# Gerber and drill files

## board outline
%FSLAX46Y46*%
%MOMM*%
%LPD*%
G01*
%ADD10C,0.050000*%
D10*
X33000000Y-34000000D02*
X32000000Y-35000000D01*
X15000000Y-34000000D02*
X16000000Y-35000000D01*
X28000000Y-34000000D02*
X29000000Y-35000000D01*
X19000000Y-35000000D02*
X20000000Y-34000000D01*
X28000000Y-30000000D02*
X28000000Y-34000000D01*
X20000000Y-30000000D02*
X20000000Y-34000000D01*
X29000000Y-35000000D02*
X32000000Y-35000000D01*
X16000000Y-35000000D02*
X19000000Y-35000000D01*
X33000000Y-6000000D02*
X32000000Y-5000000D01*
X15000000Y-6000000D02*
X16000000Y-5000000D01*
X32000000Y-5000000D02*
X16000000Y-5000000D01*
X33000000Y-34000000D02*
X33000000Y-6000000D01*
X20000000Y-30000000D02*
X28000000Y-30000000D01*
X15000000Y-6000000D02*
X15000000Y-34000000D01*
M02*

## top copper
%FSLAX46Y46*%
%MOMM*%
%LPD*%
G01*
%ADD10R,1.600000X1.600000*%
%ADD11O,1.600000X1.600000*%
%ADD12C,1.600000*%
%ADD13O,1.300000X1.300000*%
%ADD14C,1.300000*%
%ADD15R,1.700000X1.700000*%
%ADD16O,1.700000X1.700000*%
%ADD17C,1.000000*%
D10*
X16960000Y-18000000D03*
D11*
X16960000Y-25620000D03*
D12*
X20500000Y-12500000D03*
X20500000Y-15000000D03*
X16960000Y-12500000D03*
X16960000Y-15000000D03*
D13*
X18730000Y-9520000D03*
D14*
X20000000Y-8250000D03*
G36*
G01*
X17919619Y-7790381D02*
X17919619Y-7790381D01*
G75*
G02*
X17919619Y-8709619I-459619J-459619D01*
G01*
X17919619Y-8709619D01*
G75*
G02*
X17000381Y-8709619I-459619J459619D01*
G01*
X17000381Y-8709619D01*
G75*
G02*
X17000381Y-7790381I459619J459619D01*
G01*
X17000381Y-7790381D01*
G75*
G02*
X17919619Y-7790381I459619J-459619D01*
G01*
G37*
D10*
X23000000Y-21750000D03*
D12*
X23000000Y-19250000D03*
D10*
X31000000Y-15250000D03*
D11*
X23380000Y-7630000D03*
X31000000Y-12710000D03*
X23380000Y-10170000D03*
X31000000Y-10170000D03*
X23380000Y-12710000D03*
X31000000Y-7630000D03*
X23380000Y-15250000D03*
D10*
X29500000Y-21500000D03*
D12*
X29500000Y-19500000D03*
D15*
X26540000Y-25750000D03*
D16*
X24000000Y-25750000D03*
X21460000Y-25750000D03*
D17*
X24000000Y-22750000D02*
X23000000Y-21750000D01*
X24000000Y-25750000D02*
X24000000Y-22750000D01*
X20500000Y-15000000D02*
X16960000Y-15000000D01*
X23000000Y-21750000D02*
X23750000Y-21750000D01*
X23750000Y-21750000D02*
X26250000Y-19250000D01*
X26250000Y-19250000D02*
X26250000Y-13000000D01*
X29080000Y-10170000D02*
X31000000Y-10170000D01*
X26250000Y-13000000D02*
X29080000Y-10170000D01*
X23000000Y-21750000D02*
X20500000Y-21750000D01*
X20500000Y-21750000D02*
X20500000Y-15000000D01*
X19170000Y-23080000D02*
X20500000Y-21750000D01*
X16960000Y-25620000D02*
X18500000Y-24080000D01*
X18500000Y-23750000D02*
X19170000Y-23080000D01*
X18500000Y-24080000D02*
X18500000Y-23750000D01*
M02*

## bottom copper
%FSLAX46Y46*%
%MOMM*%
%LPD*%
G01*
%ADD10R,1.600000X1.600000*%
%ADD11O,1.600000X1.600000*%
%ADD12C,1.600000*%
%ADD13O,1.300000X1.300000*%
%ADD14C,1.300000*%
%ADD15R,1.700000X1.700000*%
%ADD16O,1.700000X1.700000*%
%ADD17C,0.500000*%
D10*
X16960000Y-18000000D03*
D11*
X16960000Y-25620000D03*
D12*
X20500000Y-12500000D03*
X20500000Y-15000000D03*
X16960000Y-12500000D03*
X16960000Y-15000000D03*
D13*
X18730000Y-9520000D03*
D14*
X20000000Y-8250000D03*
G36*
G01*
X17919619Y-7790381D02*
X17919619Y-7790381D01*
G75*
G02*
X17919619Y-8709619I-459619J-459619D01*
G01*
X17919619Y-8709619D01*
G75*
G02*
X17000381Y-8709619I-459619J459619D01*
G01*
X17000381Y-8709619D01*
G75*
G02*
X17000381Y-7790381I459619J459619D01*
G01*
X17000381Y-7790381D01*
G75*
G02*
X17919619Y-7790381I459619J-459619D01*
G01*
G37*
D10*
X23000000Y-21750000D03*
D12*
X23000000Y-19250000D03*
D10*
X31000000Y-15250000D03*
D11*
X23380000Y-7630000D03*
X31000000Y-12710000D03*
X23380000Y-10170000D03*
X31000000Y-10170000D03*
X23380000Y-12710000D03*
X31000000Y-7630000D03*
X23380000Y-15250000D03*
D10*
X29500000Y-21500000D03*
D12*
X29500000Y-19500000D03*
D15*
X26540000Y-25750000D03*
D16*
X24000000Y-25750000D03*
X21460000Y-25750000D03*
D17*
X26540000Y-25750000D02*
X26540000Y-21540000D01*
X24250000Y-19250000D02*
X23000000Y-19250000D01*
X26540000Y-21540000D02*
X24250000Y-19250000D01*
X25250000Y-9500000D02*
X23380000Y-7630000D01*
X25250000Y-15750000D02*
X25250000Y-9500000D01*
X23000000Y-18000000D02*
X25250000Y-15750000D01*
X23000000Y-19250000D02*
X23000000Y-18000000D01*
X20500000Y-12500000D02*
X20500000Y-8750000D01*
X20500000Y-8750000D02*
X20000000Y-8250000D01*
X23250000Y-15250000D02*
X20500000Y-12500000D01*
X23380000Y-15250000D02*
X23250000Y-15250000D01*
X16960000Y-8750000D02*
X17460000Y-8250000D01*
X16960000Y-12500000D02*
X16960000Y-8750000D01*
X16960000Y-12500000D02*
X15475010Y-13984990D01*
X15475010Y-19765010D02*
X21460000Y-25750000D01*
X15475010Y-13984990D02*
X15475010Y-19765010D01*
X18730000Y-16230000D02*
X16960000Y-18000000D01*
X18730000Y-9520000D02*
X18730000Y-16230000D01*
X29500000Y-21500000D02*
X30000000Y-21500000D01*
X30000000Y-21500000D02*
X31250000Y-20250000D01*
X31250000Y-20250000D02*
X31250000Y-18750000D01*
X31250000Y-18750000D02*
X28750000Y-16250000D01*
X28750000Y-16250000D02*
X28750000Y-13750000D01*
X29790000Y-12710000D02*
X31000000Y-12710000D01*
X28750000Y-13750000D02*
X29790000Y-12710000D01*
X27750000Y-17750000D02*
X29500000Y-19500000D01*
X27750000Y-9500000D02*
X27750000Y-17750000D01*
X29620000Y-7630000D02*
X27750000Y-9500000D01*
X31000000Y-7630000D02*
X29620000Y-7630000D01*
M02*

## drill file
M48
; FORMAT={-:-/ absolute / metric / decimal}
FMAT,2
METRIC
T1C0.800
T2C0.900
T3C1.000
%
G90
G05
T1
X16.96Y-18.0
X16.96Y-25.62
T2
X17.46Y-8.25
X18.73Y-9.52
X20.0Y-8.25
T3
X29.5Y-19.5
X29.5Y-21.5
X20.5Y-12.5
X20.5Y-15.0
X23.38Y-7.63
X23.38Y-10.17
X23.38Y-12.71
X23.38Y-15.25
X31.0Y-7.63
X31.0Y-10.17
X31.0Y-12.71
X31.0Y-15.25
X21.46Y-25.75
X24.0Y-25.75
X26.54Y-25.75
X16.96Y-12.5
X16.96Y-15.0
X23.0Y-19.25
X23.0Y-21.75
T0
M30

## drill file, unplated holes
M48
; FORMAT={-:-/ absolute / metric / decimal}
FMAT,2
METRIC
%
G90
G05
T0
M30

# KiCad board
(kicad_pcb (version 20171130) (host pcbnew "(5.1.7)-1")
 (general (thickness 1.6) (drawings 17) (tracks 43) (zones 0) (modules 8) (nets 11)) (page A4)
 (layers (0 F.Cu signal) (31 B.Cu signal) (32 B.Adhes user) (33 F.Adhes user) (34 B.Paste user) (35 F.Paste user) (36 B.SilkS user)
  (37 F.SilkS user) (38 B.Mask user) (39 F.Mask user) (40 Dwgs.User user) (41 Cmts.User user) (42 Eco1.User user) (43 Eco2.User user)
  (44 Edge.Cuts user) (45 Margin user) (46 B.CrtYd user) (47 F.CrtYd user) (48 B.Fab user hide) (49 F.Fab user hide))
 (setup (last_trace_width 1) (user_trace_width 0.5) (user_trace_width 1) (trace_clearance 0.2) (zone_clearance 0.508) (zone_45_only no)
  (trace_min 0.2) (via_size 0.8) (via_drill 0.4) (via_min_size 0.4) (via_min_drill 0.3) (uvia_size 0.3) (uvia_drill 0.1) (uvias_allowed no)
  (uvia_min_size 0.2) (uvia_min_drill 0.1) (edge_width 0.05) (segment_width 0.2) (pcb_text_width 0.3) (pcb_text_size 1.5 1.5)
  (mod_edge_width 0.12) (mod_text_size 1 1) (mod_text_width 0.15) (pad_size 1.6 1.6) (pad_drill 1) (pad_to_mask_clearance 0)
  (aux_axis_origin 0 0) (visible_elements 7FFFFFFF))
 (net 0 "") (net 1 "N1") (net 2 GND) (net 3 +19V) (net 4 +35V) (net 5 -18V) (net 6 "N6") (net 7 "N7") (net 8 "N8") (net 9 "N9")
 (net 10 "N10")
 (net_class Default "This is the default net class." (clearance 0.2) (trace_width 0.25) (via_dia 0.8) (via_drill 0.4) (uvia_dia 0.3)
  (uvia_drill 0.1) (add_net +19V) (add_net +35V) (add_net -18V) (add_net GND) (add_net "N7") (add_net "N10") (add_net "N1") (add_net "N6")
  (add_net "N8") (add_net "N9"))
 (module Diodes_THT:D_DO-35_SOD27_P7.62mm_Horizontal (layer F.Cu) (at 16.96 18 270)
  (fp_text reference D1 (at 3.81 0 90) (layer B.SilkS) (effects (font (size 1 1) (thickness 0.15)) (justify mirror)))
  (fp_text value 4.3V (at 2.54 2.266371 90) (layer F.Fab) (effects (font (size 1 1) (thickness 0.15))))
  (pad 1 thru_hole rect (at 0 0 270) (size 1.6 1.6) (drill 0.8) (layers *.Cu *.Mask) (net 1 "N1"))
  (pad 2 thru_hole oval (at 7.62 0 270) (size 1.6 1.6) (drill 0.8) (layers *.Cu *.Mask) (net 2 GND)))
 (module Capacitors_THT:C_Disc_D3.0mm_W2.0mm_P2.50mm (layer F.Cu) (at 20.5 12.5 270)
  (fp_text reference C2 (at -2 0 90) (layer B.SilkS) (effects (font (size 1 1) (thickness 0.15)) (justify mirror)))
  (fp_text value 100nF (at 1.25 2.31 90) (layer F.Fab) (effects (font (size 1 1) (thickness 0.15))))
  (pad 1 thru_hole circle (at 0 0 270) (size 1.6 1.6) (drill 1) (layers *.Cu *.Mask) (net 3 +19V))
  (pad 2 thru_hole circle (at 2.5 0 270) (size 1.6 1.6) (drill 1) (layers *.Cu *.Mask) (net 2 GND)))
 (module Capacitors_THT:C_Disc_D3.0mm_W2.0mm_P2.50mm (layer F.Cu) (at 16.96 12.5 270)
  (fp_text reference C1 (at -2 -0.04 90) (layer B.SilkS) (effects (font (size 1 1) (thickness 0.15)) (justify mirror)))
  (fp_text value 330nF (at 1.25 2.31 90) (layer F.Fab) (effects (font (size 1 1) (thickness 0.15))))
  (pad 1 thru_hole circle (at 0 0 270) (size 1.6 1.6) (drill 1) (layers *.Cu *.Mask) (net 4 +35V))
  (pad 2 thru_hole circle (at 2.5 0 270) (size 1.6 1.6) (drill 1) (layers *.Cu *.Mask) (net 2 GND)))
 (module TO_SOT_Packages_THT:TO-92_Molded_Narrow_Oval (layer F.Cu) (at 20 8.25 180)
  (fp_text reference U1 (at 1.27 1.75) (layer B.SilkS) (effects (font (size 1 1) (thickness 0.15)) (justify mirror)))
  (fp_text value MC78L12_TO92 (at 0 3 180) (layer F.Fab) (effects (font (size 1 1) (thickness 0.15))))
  (pad 2 thru_hole oval (at 1.27 -1.27 270) (size 1.3 1.3) (drill 0.9) (layers *.Cu *.Mask) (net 1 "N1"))
  (pad 1 thru_hole circle (at 0 0 225) (size 1.3 1.3) (drill 0.9) (layers *.Cu *.Mask) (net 3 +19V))
  (pad 3 thru_hole oval (at 2.54 0 225) (size 1.3 1.3) (drill 0.9) (layers *.Cu *.Mask) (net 4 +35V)))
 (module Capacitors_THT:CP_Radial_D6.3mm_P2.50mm (layer F.Cu) (at 23 21.75 90)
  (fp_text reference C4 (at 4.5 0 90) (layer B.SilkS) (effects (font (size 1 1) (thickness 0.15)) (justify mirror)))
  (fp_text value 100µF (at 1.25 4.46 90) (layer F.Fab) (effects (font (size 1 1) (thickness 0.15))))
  (pad 1 thru_hole rect (at 0 0 90) (size 1.6 1.6) (drill 1) (layers *.Cu *.Mask) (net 2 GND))
  (pad 2 thru_hole circle (at 2.5 0 90) (size 1.6 1.6) (drill 1) (layers *.Cu *.Mask) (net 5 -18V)))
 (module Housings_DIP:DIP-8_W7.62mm (layer F.Cu) (at 31 15.25 180)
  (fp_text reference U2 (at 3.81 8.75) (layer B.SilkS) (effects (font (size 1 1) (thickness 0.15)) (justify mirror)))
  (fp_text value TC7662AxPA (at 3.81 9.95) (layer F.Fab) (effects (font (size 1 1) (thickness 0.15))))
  (pad 1 thru_hole rect (at 0 0 180) (size 1.6 1.6) (drill 1) (layers *.Cu *.Mask) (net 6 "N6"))
  (pad 5 thru_hole oval (at 7.62 7.62 180) (size 1.6 1.6) (drill 1) (layers *.Cu *.Mask) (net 5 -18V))
  (pad 2 thru_hole oval (at 0 2.54 180) (size 1.6 1.6) (drill 1) (layers *.Cu *.Mask) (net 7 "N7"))
  (pad 6 thru_hole oval (at 7.62 5.08 180) (size 1.6 1.6) (drill 1) (layers *.Cu *.Mask) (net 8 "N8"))
  (pad 3 thru_hole oval (at 0 5.08 180) (size 1.6 1.6) (drill 1) (layers *.Cu *.Mask) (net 2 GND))
  (pad 7 thru_hole oval (at 7.62 2.54 180) (size 1.6 1.6) (drill 1) (layers *.Cu *.Mask) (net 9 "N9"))
  (pad 4 thru_hole oval (at 0 7.62 180) (size 1.6 1.6) (drill 1) (layers *.Cu *.Mask) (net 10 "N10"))
  (pad 8 thru_hole oval (at 7.62 0 180) (size 1.6 1.6) (drill 1) (layers *.Cu *.Mask) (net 3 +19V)))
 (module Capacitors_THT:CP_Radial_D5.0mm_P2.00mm (layer F.Cu) (at 29.5 21.5 90)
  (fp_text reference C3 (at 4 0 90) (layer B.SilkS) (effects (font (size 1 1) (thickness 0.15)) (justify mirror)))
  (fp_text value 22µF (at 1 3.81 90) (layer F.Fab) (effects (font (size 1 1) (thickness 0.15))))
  (pad 1 thru_hole rect (at 0 0 90) (size 1.6 1.6) (drill 1) (layers *.Cu *.Mask) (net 7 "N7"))
  (pad 2 thru_hole circle (at 2 0 90) (size 1.6 1.6) (drill 1) (layers *.Cu *.Mask) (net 10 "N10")))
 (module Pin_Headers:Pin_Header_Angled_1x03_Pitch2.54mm (layer F.Cu) (at 26.54 25.75 270)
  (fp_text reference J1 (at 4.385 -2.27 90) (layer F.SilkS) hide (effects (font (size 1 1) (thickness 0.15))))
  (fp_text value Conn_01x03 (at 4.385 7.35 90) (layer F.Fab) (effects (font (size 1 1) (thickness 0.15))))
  (pad 1 thru_hole rect (at 0 0 270) (size 1.7 1.7) (drill 1) (layers *.Cu *.Mask) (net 5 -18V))
  (pad 2 thru_hole oval (at 0 2.54 270) (size 1.7 1.7) (drill 1) (layers *.Cu *.Mask) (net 2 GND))
  (pad 3 thru_hole oval (at 0 5.08 270) (size 1.7 1.7) (drill 1) (layers *.Cu *.Mask) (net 4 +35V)))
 (gr_line (start 33 34) (end 32 35) (layer Edge.Cuts) (width 0.05))
 (gr_line (start 15 34) (end 16 35) (layer Edge.Cuts) (width 0.05))
 (gr_line (start 28 34) (end 29 35) (layer Edge.Cuts) (width 0.05))
 (gr_line (start 19 35) (end 20 34) (layer Edge.Cuts) (width 0.05))
 (gr_line (start 28 30) (end 28 34) (layer Edge.Cuts) (width 0.05))
 (gr_line (start 20 30) (end 20 34) (layer Edge.Cuts) (width 0.05))
 (gr_line (start 29 35) (end 32 35) (layer Edge.Cuts) (width 0.05))
 (gr_line (start 16 35) (end 19 35) (layer Edge.Cuts) (width 0.05))
 (gr_line (start 33 6) (end 32 5) (layer Edge.Cuts) (width 0.05))
 (gr_line (start 15 6) (end 16 5) (layer Edge.Cuts) (width 0.05))
 (gr_line (start 32 5) (end 16 5) (layer Edge.Cuts) (width 0.05))
 (gr_line (start 33 34) (end 33 6) (layer Edge.Cuts) (width 0.05))
 (gr_line (start 20 30) (end 28 30) (layer Edge.Cuts) (width 0.05))
 (gr_line (start 15 6) (end 15 34) (layer Edge.Cuts) (width 0.05))
 (segment (start 24 22.75) (end 23 21.75) (width 1) (layer F.Cu) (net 2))
 (segment (start 24 25.75) (end 24 22.75) (width 1) (layer F.Cu) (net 2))
 (segment (start 20.5 15) (end 16.96 15) (width 1) (layer F.Cu) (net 2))
 (segment (start 23 21.75) (end 23.75 21.75) (width 1) (layer F.Cu) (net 2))
 (segment (start 23.75 21.75) (end 26.25 19.25) (width 1) (layer F.Cu) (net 2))
 (segment (start 26.25 19.25) (end 26.25 13) (width 1) (layer F.Cu) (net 2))
 (segment (start 29.08 10.17) (end 31 10.17) (width 1) (layer F.Cu) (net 2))
 (segment (start 26.25 13) (end 29.08 10.17) (width 1) (layer F.Cu) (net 2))
 (segment (start 23 21.75) (end 20.5 21.75) (width 1) (layer F.Cu) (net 2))
 (segment (start 20.5 21.75) (end 20.5 15) (width 1) (layer F.Cu) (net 2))
 (segment (start 19.17 23.08) (end 20.5 21.75) (width 1) (layer F.Cu) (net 2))
 (segment (start 16.96 25.62) (end 18.5 24.08) (width 1) (layer F.Cu) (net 2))
 (segment (start 18.5 23.75) (end 19.17 23.08) (width 1) (layer F.Cu) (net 2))
 (segment (start 18.5 24.08) (end 18.5 23.75) (width 1) (layer F.Cu) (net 2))
 (segment (start 26.54 25.75) (end 26.54 21.54) (width 0.5) (layer B.Cu) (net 5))
 (segment (start 24.25 19.25) (end 23 19.25) (width 0.5) (layer B.Cu) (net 5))
 (segment (start 26.54 21.54) (end 24.25 19.25) (width 0.5) (layer B.Cu) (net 5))
 (segment (start 25.25 9.5) (end 23.38 7.63) (width 0.5) (layer B.Cu) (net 5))
 (segment (start 25.25 15.75) (end 25.25 9.5) (width 0.5) (layer B.Cu) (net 5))
 (segment (start 23 18) (end 25.25 15.75) (width 0.5) (layer B.Cu) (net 5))
 (segment (start 23 19.25) (end 23 18) (width 0.5) (layer B.Cu) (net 5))
 (segment (start 20.5 12.5) (end 20.5 8.75) (width 0.5) (layer B.Cu) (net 3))
 (segment (start 20.5 8.75) (end 20 8.25) (width 0.5) (layer B.Cu) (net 3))
 (segment (start 23.25 15.25) (end 20.5 12.5) (width 0.5) (layer B.Cu) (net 3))
 (segment (start 23.38 15.25) (end 23.25 15.25) (width 0.5) (layer B.Cu) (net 3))
 (segment (start 16.96 8.75) (end 17.46 8.25) (width 0.5) (layer B.Cu) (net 4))
 (segment (start 16.96 12.5) (end 16.96 8.75) (width 0.5) (layer B.Cu) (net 4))
 (segment (start 16.96 12.5) (end 15.47501 13.98499) (width 0.5) (layer B.Cu) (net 4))
 (segment (start 15.47501 19.76501) (end 21.46 25.75) (width 0.5) (layer B.Cu) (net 4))
 (segment (start 15.47501 13.98499) (end 15.47501 19.76501) (width 0.5) (layer B.Cu) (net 4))
 (segment (start 18.73 16.23) (end 16.96 18) (width 0.5) (layer B.Cu) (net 1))
 (segment (start 18.73 9.52) (end 18.73 16.23) (width 0.5) (layer B.Cu) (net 1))
 (segment (start 29.5 21.5) (end 30 21.5) (width 0.5) (layer B.Cu) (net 7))
 (segment (start 30 21.5) (end 31.25 20.25) (width 0.5) (layer B.Cu) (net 7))
 (segment (start 31.25 20.25) (end 31.25 18.75) (width 0.5) (layer B.Cu) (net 7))
 (segment (start 31.25 18.75) (end 28.75 16.25) (width 0.5) (layer B.Cu) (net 7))
 (segment (start 28.75 16.25) (end 28.75 13.75) (width 0.5) (layer B.Cu) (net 7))
 (segment (start 29.79 12.71) (end 31 12.71) (width 0.5) (layer B.Cu) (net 7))
 (segment (start 28.75 13.75) (end 29.79 12.71) (width 0.5) (layer B.Cu) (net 7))
 (segment (start 27.75 17.75) (end 29.5 19.5) (width 0.5) (layer B.Cu) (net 10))
 (segment (start 27.75 9.5) (end 27.75 17.75) (width 0.5) (layer B.Cu) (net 10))
 (segment (start 29.62 7.63) (end 27.75 9.5) (width 0.5) (layer B.Cu) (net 10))
 (segment (start 31 7.63) (end 29.62 7.63) (width 0.5) (layer B.Cu) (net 10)))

